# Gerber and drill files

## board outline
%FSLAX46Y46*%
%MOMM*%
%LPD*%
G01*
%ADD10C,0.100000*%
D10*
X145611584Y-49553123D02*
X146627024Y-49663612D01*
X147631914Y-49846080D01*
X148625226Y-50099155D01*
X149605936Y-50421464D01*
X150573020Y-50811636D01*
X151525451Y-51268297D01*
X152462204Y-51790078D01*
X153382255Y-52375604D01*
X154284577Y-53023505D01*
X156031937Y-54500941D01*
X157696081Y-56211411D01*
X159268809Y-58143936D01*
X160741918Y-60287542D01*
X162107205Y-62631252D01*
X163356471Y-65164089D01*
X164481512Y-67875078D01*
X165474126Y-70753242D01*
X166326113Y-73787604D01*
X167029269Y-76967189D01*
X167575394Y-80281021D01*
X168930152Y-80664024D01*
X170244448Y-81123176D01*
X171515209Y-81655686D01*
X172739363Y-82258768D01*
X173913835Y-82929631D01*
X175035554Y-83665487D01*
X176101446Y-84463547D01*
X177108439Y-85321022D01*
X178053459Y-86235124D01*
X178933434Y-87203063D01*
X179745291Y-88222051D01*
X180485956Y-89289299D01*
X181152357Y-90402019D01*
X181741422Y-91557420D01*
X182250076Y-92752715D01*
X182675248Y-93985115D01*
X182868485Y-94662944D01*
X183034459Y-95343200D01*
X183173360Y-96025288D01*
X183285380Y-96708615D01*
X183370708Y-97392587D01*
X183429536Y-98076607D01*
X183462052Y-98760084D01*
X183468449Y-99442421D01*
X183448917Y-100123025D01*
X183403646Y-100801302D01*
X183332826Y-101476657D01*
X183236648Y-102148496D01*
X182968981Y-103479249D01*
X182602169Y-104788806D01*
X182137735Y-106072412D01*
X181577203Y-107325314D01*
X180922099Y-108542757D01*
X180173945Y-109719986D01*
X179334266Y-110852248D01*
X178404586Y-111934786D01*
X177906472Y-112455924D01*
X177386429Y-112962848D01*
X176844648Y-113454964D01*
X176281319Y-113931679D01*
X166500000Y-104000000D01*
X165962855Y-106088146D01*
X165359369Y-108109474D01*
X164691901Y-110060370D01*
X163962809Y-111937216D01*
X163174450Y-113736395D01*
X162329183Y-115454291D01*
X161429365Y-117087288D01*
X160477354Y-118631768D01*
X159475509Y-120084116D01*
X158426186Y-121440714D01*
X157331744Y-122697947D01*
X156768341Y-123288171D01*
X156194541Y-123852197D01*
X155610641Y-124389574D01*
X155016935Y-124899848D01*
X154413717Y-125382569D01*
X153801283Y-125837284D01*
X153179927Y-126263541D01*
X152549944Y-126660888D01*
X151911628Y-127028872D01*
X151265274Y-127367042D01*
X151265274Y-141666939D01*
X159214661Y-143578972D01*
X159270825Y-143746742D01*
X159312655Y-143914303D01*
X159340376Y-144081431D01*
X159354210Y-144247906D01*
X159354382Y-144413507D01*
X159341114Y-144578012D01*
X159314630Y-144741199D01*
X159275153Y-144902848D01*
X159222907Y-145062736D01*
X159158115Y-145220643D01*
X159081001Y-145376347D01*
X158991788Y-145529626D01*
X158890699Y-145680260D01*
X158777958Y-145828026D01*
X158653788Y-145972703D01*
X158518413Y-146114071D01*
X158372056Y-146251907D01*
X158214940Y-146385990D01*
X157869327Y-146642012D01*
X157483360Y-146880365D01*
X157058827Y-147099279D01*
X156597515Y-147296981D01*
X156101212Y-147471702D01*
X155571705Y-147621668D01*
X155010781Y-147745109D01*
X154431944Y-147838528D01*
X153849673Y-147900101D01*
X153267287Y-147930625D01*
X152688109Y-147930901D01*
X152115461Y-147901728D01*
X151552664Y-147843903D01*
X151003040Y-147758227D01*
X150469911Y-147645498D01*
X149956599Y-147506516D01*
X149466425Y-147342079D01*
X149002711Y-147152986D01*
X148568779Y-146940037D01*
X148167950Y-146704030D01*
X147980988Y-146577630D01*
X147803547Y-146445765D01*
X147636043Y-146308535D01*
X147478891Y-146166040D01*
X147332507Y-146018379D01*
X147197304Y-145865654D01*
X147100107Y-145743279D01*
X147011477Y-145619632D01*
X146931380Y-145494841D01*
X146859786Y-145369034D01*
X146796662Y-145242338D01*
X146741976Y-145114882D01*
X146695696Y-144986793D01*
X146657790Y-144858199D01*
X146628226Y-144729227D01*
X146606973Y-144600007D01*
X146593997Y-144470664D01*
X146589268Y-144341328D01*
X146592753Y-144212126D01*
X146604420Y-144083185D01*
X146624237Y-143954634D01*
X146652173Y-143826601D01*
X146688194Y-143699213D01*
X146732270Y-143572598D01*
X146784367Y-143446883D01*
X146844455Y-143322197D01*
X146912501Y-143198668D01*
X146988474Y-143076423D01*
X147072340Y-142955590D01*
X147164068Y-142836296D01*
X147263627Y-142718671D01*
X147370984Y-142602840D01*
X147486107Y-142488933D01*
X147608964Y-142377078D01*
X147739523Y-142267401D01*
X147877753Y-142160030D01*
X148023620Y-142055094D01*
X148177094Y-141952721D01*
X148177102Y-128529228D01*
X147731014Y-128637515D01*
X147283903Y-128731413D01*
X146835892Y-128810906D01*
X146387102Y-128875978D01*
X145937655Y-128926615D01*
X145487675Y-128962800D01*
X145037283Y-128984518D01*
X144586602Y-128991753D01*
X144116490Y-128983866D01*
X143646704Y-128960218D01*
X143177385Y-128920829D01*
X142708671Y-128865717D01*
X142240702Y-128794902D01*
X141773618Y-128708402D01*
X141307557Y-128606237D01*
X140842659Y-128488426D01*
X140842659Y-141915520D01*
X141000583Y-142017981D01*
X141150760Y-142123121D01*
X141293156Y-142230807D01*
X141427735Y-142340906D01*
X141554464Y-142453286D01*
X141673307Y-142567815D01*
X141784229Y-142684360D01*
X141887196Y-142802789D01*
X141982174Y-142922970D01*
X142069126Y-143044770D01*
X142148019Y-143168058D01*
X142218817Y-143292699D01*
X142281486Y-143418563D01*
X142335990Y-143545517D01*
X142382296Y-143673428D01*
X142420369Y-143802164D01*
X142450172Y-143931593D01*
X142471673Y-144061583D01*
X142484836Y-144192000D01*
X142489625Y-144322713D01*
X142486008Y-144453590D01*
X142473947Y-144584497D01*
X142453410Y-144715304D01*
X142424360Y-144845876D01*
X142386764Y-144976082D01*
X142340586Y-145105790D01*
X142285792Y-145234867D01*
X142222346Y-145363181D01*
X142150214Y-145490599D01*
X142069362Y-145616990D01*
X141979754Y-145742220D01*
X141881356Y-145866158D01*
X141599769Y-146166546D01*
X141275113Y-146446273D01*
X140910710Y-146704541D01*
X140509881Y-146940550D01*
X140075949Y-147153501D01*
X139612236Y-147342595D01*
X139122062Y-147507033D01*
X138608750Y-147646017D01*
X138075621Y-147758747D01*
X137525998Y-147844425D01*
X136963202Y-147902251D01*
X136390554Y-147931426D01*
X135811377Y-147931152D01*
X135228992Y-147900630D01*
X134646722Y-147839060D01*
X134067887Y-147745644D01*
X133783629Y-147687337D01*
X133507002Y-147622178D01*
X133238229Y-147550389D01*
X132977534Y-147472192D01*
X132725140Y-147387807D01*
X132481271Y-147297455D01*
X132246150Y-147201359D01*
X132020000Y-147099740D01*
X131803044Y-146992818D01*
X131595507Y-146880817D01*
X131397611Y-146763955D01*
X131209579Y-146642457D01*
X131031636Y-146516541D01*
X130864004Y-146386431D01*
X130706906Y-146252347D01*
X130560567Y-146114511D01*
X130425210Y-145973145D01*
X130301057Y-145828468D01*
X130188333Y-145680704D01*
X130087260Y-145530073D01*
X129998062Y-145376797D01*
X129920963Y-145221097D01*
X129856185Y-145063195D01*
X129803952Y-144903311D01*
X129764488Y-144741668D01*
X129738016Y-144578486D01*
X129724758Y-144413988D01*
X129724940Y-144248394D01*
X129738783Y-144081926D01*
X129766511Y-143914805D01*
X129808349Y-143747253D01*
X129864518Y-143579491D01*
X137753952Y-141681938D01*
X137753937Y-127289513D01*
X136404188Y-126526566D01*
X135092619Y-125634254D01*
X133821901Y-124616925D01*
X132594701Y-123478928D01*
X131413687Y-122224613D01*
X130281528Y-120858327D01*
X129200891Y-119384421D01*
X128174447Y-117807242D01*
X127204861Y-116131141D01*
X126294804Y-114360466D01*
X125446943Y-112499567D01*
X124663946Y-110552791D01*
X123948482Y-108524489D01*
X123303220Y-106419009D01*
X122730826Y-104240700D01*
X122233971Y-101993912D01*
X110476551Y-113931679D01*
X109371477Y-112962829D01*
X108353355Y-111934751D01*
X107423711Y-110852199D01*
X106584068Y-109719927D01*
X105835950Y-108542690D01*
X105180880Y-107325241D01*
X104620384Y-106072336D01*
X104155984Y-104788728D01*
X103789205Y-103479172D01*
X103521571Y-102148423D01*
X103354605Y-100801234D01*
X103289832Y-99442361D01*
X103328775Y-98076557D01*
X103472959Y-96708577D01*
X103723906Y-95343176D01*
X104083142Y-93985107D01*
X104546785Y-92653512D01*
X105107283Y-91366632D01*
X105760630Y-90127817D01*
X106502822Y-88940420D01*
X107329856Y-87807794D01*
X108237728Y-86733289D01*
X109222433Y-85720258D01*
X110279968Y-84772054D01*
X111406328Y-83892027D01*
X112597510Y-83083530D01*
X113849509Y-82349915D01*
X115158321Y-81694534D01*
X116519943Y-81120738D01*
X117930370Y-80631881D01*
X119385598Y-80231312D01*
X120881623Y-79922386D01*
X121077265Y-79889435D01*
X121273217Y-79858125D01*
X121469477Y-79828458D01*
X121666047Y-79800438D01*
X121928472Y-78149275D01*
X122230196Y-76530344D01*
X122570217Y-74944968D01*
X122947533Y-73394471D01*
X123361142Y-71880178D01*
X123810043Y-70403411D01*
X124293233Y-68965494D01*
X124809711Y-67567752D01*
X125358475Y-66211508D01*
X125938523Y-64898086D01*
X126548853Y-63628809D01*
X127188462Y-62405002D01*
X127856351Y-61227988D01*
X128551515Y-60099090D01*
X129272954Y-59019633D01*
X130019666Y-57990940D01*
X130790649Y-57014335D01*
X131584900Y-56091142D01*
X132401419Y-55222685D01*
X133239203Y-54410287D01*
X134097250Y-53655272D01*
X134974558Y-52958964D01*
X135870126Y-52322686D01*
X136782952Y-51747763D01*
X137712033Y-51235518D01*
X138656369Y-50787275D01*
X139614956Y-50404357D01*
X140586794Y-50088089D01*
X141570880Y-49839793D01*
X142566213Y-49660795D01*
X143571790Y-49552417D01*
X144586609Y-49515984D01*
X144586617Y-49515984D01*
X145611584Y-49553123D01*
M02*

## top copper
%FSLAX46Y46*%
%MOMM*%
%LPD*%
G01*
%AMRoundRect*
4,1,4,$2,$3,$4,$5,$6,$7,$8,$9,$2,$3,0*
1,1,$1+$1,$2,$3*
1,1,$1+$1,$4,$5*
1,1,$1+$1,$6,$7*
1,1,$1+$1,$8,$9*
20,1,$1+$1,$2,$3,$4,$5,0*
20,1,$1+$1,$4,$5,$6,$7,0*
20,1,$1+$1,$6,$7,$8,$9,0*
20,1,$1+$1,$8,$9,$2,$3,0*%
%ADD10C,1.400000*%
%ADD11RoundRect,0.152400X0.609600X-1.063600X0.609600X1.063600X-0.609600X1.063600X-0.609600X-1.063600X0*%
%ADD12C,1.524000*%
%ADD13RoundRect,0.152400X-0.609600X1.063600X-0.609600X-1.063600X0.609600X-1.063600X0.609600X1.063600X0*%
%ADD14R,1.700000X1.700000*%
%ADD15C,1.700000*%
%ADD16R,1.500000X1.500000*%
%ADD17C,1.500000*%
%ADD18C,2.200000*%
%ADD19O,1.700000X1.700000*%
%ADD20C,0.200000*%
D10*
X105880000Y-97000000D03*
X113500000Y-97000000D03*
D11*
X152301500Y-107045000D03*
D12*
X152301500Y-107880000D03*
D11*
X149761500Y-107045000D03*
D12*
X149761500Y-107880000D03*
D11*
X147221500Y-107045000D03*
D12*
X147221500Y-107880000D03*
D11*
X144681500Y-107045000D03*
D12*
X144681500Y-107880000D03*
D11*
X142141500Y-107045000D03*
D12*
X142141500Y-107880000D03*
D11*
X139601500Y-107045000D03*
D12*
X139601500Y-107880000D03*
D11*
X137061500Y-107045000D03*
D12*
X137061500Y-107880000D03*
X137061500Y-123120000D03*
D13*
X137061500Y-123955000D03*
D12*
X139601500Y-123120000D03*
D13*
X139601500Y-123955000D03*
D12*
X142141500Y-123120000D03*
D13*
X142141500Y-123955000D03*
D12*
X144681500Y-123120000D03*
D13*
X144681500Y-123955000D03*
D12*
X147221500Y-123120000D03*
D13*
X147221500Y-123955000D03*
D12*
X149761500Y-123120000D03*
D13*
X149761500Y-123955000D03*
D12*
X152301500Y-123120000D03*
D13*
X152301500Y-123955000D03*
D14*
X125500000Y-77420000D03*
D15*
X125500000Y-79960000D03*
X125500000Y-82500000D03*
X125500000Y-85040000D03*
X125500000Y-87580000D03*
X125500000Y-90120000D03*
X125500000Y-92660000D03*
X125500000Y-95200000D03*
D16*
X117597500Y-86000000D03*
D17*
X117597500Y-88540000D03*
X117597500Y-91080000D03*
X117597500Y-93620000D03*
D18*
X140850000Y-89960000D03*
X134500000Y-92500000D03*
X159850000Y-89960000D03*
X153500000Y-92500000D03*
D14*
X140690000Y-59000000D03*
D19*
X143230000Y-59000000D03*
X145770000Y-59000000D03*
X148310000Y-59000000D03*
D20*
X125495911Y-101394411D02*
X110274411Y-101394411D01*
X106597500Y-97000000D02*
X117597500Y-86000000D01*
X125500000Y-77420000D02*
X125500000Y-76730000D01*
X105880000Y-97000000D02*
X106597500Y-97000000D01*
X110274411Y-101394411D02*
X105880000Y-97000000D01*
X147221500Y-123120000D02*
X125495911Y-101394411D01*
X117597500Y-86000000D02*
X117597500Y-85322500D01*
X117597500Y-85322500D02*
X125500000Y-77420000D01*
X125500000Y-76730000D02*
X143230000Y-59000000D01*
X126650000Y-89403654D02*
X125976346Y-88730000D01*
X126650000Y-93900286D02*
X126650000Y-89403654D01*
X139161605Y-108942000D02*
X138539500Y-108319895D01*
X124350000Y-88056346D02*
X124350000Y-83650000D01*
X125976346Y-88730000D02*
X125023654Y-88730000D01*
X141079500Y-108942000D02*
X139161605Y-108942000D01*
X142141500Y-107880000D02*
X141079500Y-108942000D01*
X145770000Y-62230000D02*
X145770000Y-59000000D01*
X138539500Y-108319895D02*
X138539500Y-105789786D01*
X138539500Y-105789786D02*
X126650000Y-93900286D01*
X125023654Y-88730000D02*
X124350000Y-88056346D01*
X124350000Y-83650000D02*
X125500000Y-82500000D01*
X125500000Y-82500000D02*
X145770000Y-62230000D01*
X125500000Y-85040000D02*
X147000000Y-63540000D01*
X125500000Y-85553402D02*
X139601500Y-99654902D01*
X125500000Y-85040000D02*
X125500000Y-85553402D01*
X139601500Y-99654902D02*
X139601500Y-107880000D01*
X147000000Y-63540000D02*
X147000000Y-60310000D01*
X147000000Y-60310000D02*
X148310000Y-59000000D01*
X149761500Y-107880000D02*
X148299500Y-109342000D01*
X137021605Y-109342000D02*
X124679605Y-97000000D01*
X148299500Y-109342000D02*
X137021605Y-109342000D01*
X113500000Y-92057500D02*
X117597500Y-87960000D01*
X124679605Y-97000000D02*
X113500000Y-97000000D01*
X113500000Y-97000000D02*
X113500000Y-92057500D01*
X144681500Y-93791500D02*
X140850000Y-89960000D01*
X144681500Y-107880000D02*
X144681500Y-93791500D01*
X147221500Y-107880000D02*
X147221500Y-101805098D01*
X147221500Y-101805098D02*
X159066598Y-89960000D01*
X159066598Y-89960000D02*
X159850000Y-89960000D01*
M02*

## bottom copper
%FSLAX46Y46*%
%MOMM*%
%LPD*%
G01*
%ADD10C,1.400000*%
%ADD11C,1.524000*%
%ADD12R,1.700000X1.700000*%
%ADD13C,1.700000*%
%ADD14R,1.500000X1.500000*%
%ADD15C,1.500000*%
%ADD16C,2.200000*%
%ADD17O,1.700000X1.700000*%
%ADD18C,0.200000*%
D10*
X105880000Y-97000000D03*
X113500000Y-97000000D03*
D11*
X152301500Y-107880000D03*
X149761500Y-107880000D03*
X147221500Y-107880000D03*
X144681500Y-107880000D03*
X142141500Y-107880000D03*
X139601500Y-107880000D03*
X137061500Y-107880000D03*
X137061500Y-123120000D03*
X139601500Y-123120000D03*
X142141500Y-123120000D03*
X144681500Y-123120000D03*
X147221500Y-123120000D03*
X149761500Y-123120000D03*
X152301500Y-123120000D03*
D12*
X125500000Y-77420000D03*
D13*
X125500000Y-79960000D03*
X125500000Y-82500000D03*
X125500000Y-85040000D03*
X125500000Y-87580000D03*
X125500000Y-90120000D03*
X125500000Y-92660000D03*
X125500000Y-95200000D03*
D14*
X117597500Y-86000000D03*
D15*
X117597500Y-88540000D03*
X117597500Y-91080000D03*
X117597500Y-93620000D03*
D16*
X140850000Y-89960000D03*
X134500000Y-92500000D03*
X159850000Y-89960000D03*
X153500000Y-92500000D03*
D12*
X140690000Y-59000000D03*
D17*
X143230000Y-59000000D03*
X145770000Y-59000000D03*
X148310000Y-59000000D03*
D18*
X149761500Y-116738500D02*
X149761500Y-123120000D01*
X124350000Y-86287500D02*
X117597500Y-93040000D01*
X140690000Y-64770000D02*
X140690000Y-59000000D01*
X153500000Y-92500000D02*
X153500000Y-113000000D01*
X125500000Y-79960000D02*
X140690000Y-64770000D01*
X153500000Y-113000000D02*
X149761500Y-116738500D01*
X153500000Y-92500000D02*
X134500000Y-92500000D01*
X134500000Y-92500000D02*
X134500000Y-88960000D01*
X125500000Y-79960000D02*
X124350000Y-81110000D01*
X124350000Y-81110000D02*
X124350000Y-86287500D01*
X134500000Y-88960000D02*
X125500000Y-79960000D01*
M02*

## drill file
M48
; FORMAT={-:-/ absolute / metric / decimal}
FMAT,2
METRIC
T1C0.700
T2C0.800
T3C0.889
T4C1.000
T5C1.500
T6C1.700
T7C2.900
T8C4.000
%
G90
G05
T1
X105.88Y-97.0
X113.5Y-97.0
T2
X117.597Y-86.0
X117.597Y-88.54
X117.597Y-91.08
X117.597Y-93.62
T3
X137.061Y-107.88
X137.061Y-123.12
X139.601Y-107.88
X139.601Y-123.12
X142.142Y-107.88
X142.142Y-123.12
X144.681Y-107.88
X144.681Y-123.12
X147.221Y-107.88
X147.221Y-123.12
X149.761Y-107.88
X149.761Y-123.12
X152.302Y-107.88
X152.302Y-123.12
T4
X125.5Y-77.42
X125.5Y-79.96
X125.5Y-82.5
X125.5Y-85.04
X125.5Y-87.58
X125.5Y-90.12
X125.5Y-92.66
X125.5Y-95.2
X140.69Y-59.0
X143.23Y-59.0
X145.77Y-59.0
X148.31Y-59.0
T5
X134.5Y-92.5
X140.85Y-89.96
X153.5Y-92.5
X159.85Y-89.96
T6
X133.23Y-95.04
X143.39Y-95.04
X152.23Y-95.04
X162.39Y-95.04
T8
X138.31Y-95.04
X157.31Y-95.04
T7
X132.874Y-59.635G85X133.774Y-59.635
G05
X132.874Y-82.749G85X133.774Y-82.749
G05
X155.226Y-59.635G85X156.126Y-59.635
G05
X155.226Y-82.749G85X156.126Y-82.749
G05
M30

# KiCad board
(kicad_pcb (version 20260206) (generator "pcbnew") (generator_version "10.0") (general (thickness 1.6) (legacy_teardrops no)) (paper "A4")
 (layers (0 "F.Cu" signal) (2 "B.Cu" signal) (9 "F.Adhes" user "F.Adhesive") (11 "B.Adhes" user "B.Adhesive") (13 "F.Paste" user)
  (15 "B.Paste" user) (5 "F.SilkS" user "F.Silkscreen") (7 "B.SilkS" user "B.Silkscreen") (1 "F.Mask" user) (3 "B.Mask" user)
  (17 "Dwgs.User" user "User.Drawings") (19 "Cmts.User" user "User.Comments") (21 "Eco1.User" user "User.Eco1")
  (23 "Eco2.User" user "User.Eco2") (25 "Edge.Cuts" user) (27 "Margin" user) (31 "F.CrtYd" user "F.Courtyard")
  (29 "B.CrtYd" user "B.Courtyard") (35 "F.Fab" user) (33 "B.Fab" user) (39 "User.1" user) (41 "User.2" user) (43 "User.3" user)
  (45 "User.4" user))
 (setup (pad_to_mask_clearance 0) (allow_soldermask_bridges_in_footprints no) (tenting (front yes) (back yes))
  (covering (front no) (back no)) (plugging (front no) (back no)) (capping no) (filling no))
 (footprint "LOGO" (layer "F.Cu") (at 143 97)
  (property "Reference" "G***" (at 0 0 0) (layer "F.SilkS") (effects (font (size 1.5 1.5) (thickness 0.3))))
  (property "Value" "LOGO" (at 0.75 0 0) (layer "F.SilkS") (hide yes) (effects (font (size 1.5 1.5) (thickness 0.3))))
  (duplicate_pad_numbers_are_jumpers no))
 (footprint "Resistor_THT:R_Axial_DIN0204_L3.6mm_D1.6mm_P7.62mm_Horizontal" (layer "F.Cu") (at 105.88 97)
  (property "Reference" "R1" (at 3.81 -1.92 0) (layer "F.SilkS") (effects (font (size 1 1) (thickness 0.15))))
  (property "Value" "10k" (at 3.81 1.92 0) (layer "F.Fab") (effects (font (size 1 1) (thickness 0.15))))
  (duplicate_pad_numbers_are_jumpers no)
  (pad "1" thru_hole circle (at 0 0) (size 1.4 1.4) (drill 0.7) (layers "*.Cu" "*.Mask") (remove_unused_layers no) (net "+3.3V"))
  (pad "2" thru_hole circle (at 7.62 0) (size 1.4 1.4) (drill 0.7) (layers "*.Cu" "*.Mask") (remove_unused_layers no) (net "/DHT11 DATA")))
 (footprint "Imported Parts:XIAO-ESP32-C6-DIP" (layer "F.Cu") (at 144.6815 115.5)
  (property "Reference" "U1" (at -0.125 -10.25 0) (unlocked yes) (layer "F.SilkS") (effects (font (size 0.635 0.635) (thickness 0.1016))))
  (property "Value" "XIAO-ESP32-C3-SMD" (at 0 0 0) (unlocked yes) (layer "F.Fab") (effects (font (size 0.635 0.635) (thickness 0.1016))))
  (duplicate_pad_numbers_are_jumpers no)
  (pad "1" smd roundrect (at 7.62 -8.455 90) (size 2.432 1.524) (layers "F.Cu" "F.Mask") (roundrect_rratio 0.1)
   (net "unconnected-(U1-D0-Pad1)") (thermal_bridge_angle 45))
  (pad "1" thru_hole circle (at 7.62 -7.62 90) (size 1.524 1.524) (drill 0.889) (layers "*.Cu" "*.Mask") (remove_unused_layers no)
   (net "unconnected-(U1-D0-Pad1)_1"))
  (pad "2" smd roundrect (at 5.08 -8.455 90) (size 2.432 1.524) (layers "F.Cu" "F.Mask") (roundrect_rratio 0.1) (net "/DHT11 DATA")
   (thermal_bridge_angle 45))
  (pad "2" thru_hole circle (at 5.08 -7.62 90) (size 1.524 1.524) (drill 0.889) (layers "*.Cu" "*.Mask") (remove_unused_layers no)
   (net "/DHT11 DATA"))
  (pad "3" smd roundrect (at 2.54 -8.455 90) (size 2.432 1.524) (layers "F.Cu" "F.Mask") (roundrect_rratio 0.1) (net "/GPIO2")
   (thermal_bridge_angle 45))
  (pad "3" thru_hole circle (at 2.54 -7.62 90) (size 1.524 1.524) (drill 0.889) (layers "*.Cu" "*.Mask") (remove_unused_layers no)
   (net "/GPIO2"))
  (pad "4" smd roundrect (at 0 -8.455 90) (size 2.432 1.524) (layers "F.Cu" "F.Mask") (roundrect_rratio 0.1) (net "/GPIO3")
   (thermal_bridge_angle 45))
  (pad "4" thru_hole circle (at 0 -7.62 90) (size 1.524 1.524) (drill 0.889) (layers "*.Cu" "*.Mask") (remove_unused_layers no)
   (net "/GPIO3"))
  (pad "5" smd roundrect (at -2.54 -8.455 90) (size 2.432 1.524) (layers "F.Cu" "F.Mask") (roundrect_rratio 0.1) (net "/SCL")
   (thermal_bridge_angle 45))
  (pad "5" thru_hole circle (at -2.54 -7.62 90) (size 1.524 1.524) (drill 0.889) (layers "*.Cu" "*.Mask") (remove_unused_layers no)
   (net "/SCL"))
  (pad "6" smd roundrect (at -5.08 -8.455 90) (size 2.432 1.524) (layers "F.Cu" "F.Mask") (roundrect_rratio 0.1) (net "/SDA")
   (thermal_bridge_angle 45))
  (pad "6" thru_hole circle (at -5.08 -7.62 90) (size 1.524 1.524) (drill 0.889) (layers "*.Cu" "*.Mask") (remove_unused_layers no)
   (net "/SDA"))
  (pad "7" smd roundrect (at -7.62 -8.455 90) (size 2.432 1.524) (layers "F.Cu" "F.Mask") (roundrect_rratio 0.1)
   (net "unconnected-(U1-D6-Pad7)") (thermal_bridge_angle 45))
  (pad "7" thru_hole circle (at -7.62 -7.62 90) (size 1.524 1.524) (drill 0.889) (layers "*.Cu" "*.Mask") (remove_unused_layers no)
   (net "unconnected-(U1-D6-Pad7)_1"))
  (pad "8" thru_hole circle (at -7.62 7.62 270) (size 1.524 1.524) (drill 0.889) (layers "*.Cu" "*.Mask") (remove_unused_layers no)
   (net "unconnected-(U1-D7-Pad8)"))
  (pad "8" smd roundrect (at -7.62 8.455 270) (size 2.432 1.524) (layers "F.Cu" "F.Mask") (roundrect_rratio 0.1)
   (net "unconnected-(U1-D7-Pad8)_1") (thermal_bridge_angle 45))
  (pad "9" thru_hole circle (at -5.08 7.62 270) (size 1.524 1.524) (drill 0.889) (layers "*.Cu" "*.Mask") (remove_unused_layers no)
   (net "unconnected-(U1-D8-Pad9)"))
  (pad "9" smd roundrect (at -5.08 8.455 270) (size 2.432 1.524) (layers "F.Cu" "F.Mask") (roundrect_rratio 0.1)
   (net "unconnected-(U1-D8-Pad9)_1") (thermal_bridge_angle 45))
  (pad "10" thru_hole circle (at -2.54 7.62 270) (size 1.524 1.524) (drill 0.889) (layers "*.Cu" "*.Mask") (remove_unused_layers no)
   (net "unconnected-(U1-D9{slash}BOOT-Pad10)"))
  (pad "10" smd roundrect (at -2.54 8.455 270) (size 2.432 1.524) (layers "F.Cu" "F.Mask") (roundrect_rratio 0.1)
   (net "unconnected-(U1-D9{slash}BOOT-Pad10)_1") (thermal_bridge_angle 45))
  (pad "11" thru_hole circle (at 0 7.62 270) (size 1.524 1.524) (drill 0.889) (layers "*.Cu" "*.Mask") (remove_unused_layers no)
   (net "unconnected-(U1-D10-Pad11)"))
  (pad "11" smd roundrect (at 0 8.455 270) (size 2.432 1.524) (layers "F.Cu" "F.Mask") (roundrect_rratio 0.1)
   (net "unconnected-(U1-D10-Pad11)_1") (thermal_bridge_angle 45))
  (pad "12" thru_hole circle (at 2.54 7.62 270) (size 1.524 1.524) (drill 0.889) (layers "*.Cu" "*.Mask") (remove_unused_layers no)
   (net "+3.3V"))
  (pad "12" smd roundrect (at 2.54 8.455 270) (size 2.432 1.524) (layers "F.Cu" "F.Mask") (roundrect_rratio 0.1) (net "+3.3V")
   (thermal_bridge_angle 45))
  (pad "13" thru_hole circle (at 5.08 7.62 270) (size 1.524 1.524) (drill 0.889) (layers "*.Cu" "*.Mask") (remove_unused_layers no)
   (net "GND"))
  (pad "13" smd roundrect (at 5.08 8.455 270) (size 2.432 1.524) (layers "F.Cu" "F.Mask") (roundrect_rratio 0.1) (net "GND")
   (thermal_bridge_angle 45))
  (pad "14" thru_hole circle (at 7.62 7.62 270) (size 1.524 1.524) (drill 0.889) (layers "*.Cu" "*.Mask") (remove_unused_layers no)
   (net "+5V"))
  (pad "14" smd roundrect (at 7.62 8.455 270) (size 2.432 1.524) (layers "F.Cu" "F.Mask") (roundrect_rratio 0.1) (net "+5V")
   (thermal_bridge_angle 45)))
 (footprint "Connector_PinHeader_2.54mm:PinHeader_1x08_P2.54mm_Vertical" (layer "F.Cu") (at 125.5 77.42)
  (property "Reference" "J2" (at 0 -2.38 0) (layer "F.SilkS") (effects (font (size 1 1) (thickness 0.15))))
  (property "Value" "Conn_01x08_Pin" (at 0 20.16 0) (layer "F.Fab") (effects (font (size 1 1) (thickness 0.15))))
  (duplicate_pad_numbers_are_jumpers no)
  (pad "1" thru_hole rect (at 0 0) (size 1.7 1.7) (drill 1) (layers "*.Cu" "*.Mask") (remove_unused_layers no) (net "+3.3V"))
  (pad "2" thru_hole circle (at 0 2.54) (size 1.7 1.7) (drill 1) (layers "*.Cu" "*.Mask") (remove_unused_layers no) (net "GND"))
  (pad "3" thru_hole circle (at 0 5.08) (size 1.7 1.7) (drill 1) (layers "*.Cu" "*.Mask") (remove_unused_layers no) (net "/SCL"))
  (pad "4" thru_hole circle (at 0 7.62) (size 1.7 1.7) (drill 1) (layers "*.Cu" "*.Mask") (remove_unused_layers no) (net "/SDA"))
  (pad "5" thru_hole circle (at 0 10.16) (size 1.7 1.7) (drill 1) (layers "*.Cu" "*.Mask") (remove_unused_layers no)
   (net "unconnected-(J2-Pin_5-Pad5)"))
  (pad "6" thru_hole circle (at 0 12.7) (size 1.7 1.7) (drill 1) (layers "*.Cu" "*.Mask") (remove_unused_layers no)
   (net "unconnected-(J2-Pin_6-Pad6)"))
  (pad "7" thru_hole circle (at 0 15.24) (size 1.7 1.7) (drill 1) (layers "*.Cu" "*.Mask") (remove_unused_layers no)
   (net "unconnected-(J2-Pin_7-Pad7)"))
  (pad "8" thru_hole circle (at 0 17.78) (size 1.7 1.7) (drill 1) (layers "*.Cu" "*.Mask") (remove_unused_layers no)
   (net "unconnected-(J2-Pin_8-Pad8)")))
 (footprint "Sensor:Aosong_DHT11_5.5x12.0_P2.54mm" (layer "F.Cu") (at 117.5975 86)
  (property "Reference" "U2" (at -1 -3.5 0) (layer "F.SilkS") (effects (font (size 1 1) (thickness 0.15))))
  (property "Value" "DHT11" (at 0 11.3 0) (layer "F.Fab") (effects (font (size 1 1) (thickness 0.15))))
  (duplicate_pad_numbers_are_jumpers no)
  (pad "1" thru_hole rect (at 0 0) (size 1.5 1.5) (drill 0.8) (layers "*.Cu" "*.Mask") (remove_unused_layers no) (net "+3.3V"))
  (pad "2" thru_hole circle (at 0 2.54) (size 1.5 1.5) (drill 0.8) (layers "*.Cu" "*.Mask") (remove_unused_layers no) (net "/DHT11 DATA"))
  (pad "3" thru_hole circle (at 0 5.08) (size 1.5 1.5) (drill 0.8) (layers "*.Cu" "*.Mask") (remove_unused_layers no)
   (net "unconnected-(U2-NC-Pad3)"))
  (pad "4" thru_hole circle (at 0 7.62) (size 1.5 1.5) (drill 0.8) (layers "*.Cu" "*.Mask") (remove_unused_layers no) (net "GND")))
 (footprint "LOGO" (layer "F.Cu") (at 142.5 98.5)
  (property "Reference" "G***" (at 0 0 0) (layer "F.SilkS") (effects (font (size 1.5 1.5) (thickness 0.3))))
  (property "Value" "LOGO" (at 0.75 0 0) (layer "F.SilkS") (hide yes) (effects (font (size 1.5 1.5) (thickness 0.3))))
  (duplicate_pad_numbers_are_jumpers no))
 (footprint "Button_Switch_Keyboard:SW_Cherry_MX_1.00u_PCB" (layer "F.Cu") (at 140.85 89.96)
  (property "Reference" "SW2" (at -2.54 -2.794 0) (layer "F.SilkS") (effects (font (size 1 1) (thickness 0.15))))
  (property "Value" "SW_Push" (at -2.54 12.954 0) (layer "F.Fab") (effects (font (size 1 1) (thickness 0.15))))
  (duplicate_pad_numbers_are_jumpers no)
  (pad "" np_thru_hole circle (at -7.62 5.08) (size 1.7 1.7) (drill 1.7) (layers "*.Cu" "*.Mask"))
  (pad "" np_thru_hole circle (at -2.54 5.08) (size 4 4) (drill 4) (layers "*.Cu" "*.Mask"))
  (pad "" np_thru_hole circle (at 2.54 5.08) (size 1.7 1.7) (drill 1.7) (layers "*.Cu" "*.Mask"))
  (pad "1" thru_hole circle (at 0 0) (size 2.2 2.2) (drill 1.5) (layers "*.Cu" "*.Mask") (remove_unused_layers no) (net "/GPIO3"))
  (pad "2" thru_hole circle (at -6.35 2.54) (size 2.2 2.2) (drill 1.5) (layers "*.Cu" "*.Mask") (remove_unused_layers no) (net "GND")))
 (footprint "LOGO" (layer "F.Cu") (at 143 98.5)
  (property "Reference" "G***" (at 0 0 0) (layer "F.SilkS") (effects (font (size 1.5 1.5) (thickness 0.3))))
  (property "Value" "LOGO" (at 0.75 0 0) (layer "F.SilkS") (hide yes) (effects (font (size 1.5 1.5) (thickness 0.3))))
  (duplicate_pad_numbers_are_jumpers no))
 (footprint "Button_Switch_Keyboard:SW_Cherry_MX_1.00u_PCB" (layer "F.Cu") (at 159.85 89.96)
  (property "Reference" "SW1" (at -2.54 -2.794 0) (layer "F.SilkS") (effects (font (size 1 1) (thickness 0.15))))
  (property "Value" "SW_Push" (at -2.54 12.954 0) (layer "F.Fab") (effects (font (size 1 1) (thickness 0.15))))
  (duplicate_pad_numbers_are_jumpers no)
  (pad "" np_thru_hole circle (at -7.62 5.08) (size 1.7 1.7) (drill 1.7) (layers "*.Cu" "*.Mask"))
  (pad "" np_thru_hole circle (at -2.54 5.08) (size 4 4) (drill 4) (layers "*.Cu" "*.Mask"))
  (pad "" np_thru_hole circle (at 2.54 5.08) (size 1.7 1.7) (drill 1.7) (layers "*.Cu" "*.Mask"))
  (pad "1" thru_hole circle (at 0 0) (size 2.2 2.2) (drill 1.5) (layers "*.Cu" "*.Mask") (remove_unused_layers no) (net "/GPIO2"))
  (pad "2" thru_hole circle (at -6.35 2.54) (size 2.2 2.2) (drill 1.5) (layers "*.Cu" "*.Mask") (remove_unused_layers no) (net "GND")))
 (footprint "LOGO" (layer "F.Cu") (at 142.5 97.5)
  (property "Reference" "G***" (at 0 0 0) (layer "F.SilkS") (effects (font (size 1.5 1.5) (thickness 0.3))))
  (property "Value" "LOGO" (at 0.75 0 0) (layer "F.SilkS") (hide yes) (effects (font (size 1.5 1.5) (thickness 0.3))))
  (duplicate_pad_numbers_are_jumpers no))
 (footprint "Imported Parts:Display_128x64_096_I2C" (layer "F.Cu") (at 144.5 59)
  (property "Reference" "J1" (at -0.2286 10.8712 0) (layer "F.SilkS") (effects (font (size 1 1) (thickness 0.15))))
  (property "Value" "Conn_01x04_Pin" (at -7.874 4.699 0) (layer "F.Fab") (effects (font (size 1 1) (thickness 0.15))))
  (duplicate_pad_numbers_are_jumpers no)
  (pad "" np_thru_hole oval (at -11.176 0.635) (size 3.8 2.9) (drill oval 3.8 2.9) (layers "*.Cu" "*.Mask"))
  (pad "" np_thru_hole oval (at -11.176 23.749) (size 3.8 2.9) (drill oval 3.8 2.9) (layers "*.Cu" "*.Mask"))
  (pad "" np_thru_hole oval (at 11.176 0.635) (size 3.8 2.9) (drill oval 3.8 2.9) (layers "*.Cu" "*.Mask"))
  (pad "" np_thru_hole oval (at 11.176 23.749) (size 3.8 2.9) (drill oval 3.8 2.9) (layers "*.Cu" "*.Mask"))
  (pad "1" thru_hole rect (at -3.81 0 90) (size 1.7 1.7) (drill 1) (layers "*.Cu" "*.Mask") (remove_unused_layers no) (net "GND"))
  (pad "2" thru_hole oval (at -1.27 0 90) (size 1.7 1.7) (drill 1) (layers "*.Cu" "*.Mask") (remove_unused_layers no) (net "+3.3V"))
  (pad "3" thru_hole oval (at 1.27 0 90) (size 1.7 1.7) (drill 1) (layers "*.Cu" "*.Mask") (remove_unused_layers no) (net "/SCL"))
  (pad "4" thru_hole oval (at 3.81 0 90) (size 1.7 1.7) (drill 1) (layers "*.Cu" "*.Mask") (remove_unused_layers no) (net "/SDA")))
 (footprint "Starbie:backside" (layer "B.Cu") (at 145 96.5 180)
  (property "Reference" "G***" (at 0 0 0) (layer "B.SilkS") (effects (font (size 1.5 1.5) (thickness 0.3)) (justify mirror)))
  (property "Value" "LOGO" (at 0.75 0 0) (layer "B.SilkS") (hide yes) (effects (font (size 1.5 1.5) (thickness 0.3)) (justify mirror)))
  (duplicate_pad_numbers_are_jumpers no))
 (gr_poly
  (pts (xy 145.611584 49.553123) (xy 146.627024 49.663612) (xy 147.631914 49.84608) (xy 148.625226 50.099155) (xy 149.605936 50.421464)
   (xy 150.57302 50.811636) (xy 151.525451 51.268297) (xy 152.462204 51.790078) (xy 153.382255 52.375604) (xy 154.284577 53.023505)
   (xy 156.031937 54.500941) (xy 157.696081 56.211411) (xy 159.268809 58.143936) (xy 160.741918 60.287542) (xy 162.107205 62.631252)
   (xy 163.356471 65.164089) (xy 164.481512 67.875078) (xy 165.474126 70.753242) (xy 166.326113 73.787604) (xy 167.029269 76.967189)
   (xy 167.575394 80.281021) (xy 168.930152 80.664024) (xy 170.244448 81.123176) (xy 171.515209 81.655686) (xy 172.739363 82.258768)
   (xy 173.913835 82.929631) (xy 175.035554 83.665487) (xy 176.101446 84.463547) (xy 177.108439 85.321022) (xy 178.053459 86.235124)
   (xy 178.933434 87.203063) (xy 179.745291 88.222051) (xy 180.485956 89.289299) (xy 181.152357 90.402019) (xy 181.741422 91.55742)
   (xy 182.250076 92.752715) (xy 182.675248 93.985115) (xy 182.868485 94.662944) (xy 183.034459 95.3432) (xy 183.17336 96.025288)
   (xy 183.28538 96.708615) (xy 183.370708 97.392587) (xy 183.429536 98.076607) (xy 183.462052 98.760084) (xy 183.468449 99.442421)
   (xy 183.448917 100.123025) (xy 183.403646 100.801302) (xy 183.332826 101.476657) (xy 183.236648 102.148496) (xy 182.968981 103.479249)
   (xy 182.602169 104.788806) (xy 182.137735 106.072412) (xy 181.577203 107.325314) (xy 180.922099 108.542757) (xy 180.173945 109.719986)
   (xy 179.334266 110.852248) (xy 178.404586 111.934786) (xy 177.906472 112.455924) (xy 177.386429 112.962848) (xy 176.844648 113.454964)
   (xy 176.281319 113.931679) (xy 166.5 104) (xy 165.962855 106.088146) (xy 165.359369 108.109474) (xy 164.691901 110.06037)
   (xy 163.962809 111.937216) (xy 163.17445 113.736395) (xy 162.329183 115.454291) (xy 161.429365 117.087288) (xy 160.477354 118.631768)
   (xy 159.475509 120.084116) (xy 158.426186 121.440714) (xy 157.331744 122.697947) (xy 156.768341 123.288171) (xy 156.194541 123.852197)
   (xy 155.610641 124.389574) (xy 155.016935 124.899848) (xy 154.413717 125.382569) (xy 153.801283 125.837284) (xy 153.179927 126.263541)
   (xy 152.549944 126.660888) (xy 151.911628 127.028872) (xy 151.265274 127.367042) (xy 151.265274 141.666939) (xy 159.214661 143.578972)
   (xy 159.270825 143.746742) (xy 159.312655 143.914303) (xy 159.340376 144.081431) (xy 159.35421 144.247906) (xy 159.354382 144.413507)
   (xy 159.341114 144.578012) (xy 159.31463 144.741199) (xy 159.275153 144.902848) (xy 159.222907 145.062736) (xy 159.158115 145.220643)
   (xy 159.081001 145.376347) (xy 158.991788 145.529626) (xy 158.890699 145.68026) (xy 158.777958 145.828026) (xy 158.653788 145.972703)
   (xy 158.518413 146.114071) (xy 158.372056 146.251907) (xy 158.21494 146.38599) (xy 157.869327 146.642012) (xy 157.48336 146.880365)
   (xy 157.058827 147.099279) (xy 156.597515 147.296981) (xy 156.101212 147.471702) (xy 155.571705 147.621668) (xy 155.010781 147.745109)
   (xy 154.431944 147.838528) (xy 153.849673 147.900101) (xy 153.267287 147.930625) (xy 152.688109 147.930901) (xy 152.115461 147.901728)
   (xy 151.552664 147.843903) (xy 151.00304 147.758227) (xy 150.469911 147.645498) (xy 149.956599 147.506516) (xy 149.466425 147.342079)
   (xy 149.002711 147.152986) (xy 148.568779 146.940037) (xy 148.16795 146.70403) (xy 147.980988 146.57763) (xy 147.803547 146.445765)
   (xy 147.636043 146.308535) (xy 147.478891 146.16604) (xy 147.332507 146.018379) (xy 147.197304 145.865654) (xy 147.100107 145.743279)
   (xy 147.011477 145.619632) (xy 146.93138 145.494841) (xy 146.859786 145.369034) (xy 146.796662 145.242338) (xy 146.741976 145.114882)
   (xy 146.695696 144.986793) (xy 146.65779 144.858199) (xy 146.628226 144.729227) (xy 146.606973 144.600007) (xy 146.593997 144.470664)
   (xy 146.589268 144.341328) (xy 146.592753 144.212126) (xy 146.60442 144.083185) (xy 146.624237 143.954634) (xy 146.652173 143.826601)
   (xy 146.688194 143.699213) (xy 146.73227 143.572598) (xy 146.784367 143.446883) (xy 146.844455 143.322197) (xy 146.912501 143.198668)
   (xy 146.988474 143.076423) (xy 147.07234 142.95559) (xy 147.164068 142.836296) (xy 147.263627 142.718671) (xy 147.370984 142.60284)
   (xy 147.486107 142.488933) (xy 147.608964 142.377078) (xy 147.739523 142.267401) (xy 147.877753 142.16003) (xy 148.02362 142.055094)
   (xy 148.177094 141.952721) (xy 148.177102 128.529228) (xy 147.731014 128.637515) (xy 147.283903 128.731413) (xy 146.835892 128.810906)
   (xy 146.387102 128.875978) (xy 145.937655 128.926615) (xy 145.487675 128.9628) (xy 145.037283 128.984518) (xy 144.586602 128.991753)
   (xy 144.11649 128.983866) (xy 143.646704 128.960218) (xy 143.177385 128.920829) (xy 142.708671 128.865717) (xy 142.240702 128.794902)
   (xy 141.773618 128.708402) (xy 141.307557 128.606237) (xy 140.842659 128.488426) (xy 140.842659 141.91552) (xy 141.000583 142.017981)
   (xy 141.15076 142.123121) (xy 141.293156 142.230807) (xy 141.427735 142.340906) (xy 141.554464 142.453286) (xy 141.673307 142.567815)
   (xy 141.784229 142.68436) (xy 141.887196 142.802789) (xy 141.982174 142.92297) (xy 142.069126 143.04477) (xy 142.148019 143.168058)
   (xy 142.218817 143.292699) (xy 142.281486 143.418563) (xy 142.33599 143.545517) (xy 142.382296 143.673428) (xy 142.420369 143.802164)
   (xy 142.450172 143.931593) (xy 142.471673 144.061583) (xy 142.484836 144.192) (xy 142.489625 144.322713) (xy 142.486008 144.45359)
   (xy 142.473947 144.584497) (xy 142.45341 144.715304) (xy 142.42436 144.845876) (xy 142.386764 144.976082) (xy 142.340586 145.10579)
   (xy 142.285792 145.234867) (xy 142.222346 145.363181) (xy 142.150214 145.490599) (xy 142.069362 145.61699) (xy 141.979754 145.74222)
   (xy 141.881356 145.866158) (xy 141.599769 146.166546) (xy 141.275113 146.446273) (xy 140.91071 146.704541) (xy 140.509881 146.94055)
   (xy 140.075949 147.153501) (xy 139.612236 147.342595) (xy 139.122062 147.507033) (xy 138.60875 147.646017) (xy 138.075621 147.758747)
   (xy 137.525998 147.844425) (xy 136.963202 147.902251) (xy 136.390554 147.931426) (xy 135.811377 147.931152) (xy 135.228992 147.90063)
   (xy 134.646722 147.83906) (xy 134.067887 147.745644) (xy 133.783629 147.687337) (xy 133.507002 147.622178) (xy 133.238229 147.550389)
   (xy 132.977534 147.472192) (xy 132.72514 147.387807) (xy 132.481271 147.297455) (xy 132.24615 147.201359) (xy 132.02 147.09974)
   (xy 131.803044 146.992818) (xy 131.595507 146.880817) (xy 131.397611 146.763955) (xy 131.209579 146.642457) (xy 131.031636 146.516541)
   (xy 130.864004 146.386431) (xy 130.706906 146.252347) (xy 130.560567 146.114511) (xy 130.42521 145.973145) (xy 130.301057 145.828468)
   (xy 130.188333 145.680704) (xy 130.08726 145.530073) (xy 129.998062 145.376797) (xy 129.920963 145.221097) (xy 129.856185 145.063195)
   (xy 129.803952 144.903311) (xy 129.764488 144.741668) (xy 129.738016 144.578486) (xy 129.724758 144.413988) (xy 129.72494 144.248394)
   (xy 129.738783 144.081926) (xy 129.766511 143.914805) (xy 129.808349 143.747253) (xy 129.864518 143.579491) (xy 137.753952 141.681938)
   (xy 137.753937 127.289513) (xy 136.404188 126.526566) (xy 135.092619 125.634254) (xy 133.821901 124.616925) (xy 132.594701 123.478928)
   (xy 131.413687 122.224613) (xy 130.281528 120.858327) (xy 129.200891 119.384421) (xy 128.174447 117.807242) (xy 127.204861 116.131141)
   (xy 126.294804 114.360466) (xy 125.446943 112.499567) (xy 124.663946 110.552791) (xy 123.948482 108.524489) (xy 123.30322 106.419009)
   (xy 122.730826 104.2407) (xy 122.233971 101.993912) (xy 110.476551 113.931679) (xy 109.371477 112.962829) (xy 108.353355 111.934751)
   (xy 107.423711 110.852199) (xy 106.584068 109.719927) (xy 105.83595 108.54269) (xy 105.18088 107.325241) (xy 104.620384 106.072336)
   (xy 104.155984 104.788728) (xy 103.789205 103.479172) (xy 103.521571 102.148423) (xy 103.354605 100.801234) (xy 103.289832 99.442361)
   (xy 103.328775 98.076557) (xy 103.472959 96.708577) (xy 103.723906 95.343176) (xy 104.083142 93.985107) (xy 104.546785 92.653512)
   (xy 105.107283 91.366632) (xy 105.76063 90.127817) (xy 106.502822 88.94042) (xy 107.329856 87.807794) (xy 108.237728 86.733289)
   (xy 109.222433 85.720258) (xy 110.279968 84.772054) (xy 111.406328 83.892027) (xy 112.59751 83.08353) (xy 113.849509 82.349915)
   (xy 115.158321 81.694534) (xy 116.519943 81.120738) (xy 117.93037 80.631881) (xy 119.385598 80.231312) (xy 120.881623 79.922386)
   (xy 121.077265 79.889435) (xy 121.273217 79.858125) (xy 121.469477 79.828458) (xy 121.666047 79.800438) (xy 121.928472 78.149275)
   (xy 122.230196 76.530344) (xy 122.570217 74.944968) (xy 122.947533 73.394471) (xy 123.361142 71.880178) (xy 123.810043 70.403411)
   (xy 124.293233 68.965494) (xy 124.809711 67.567752) (xy 125.358475 66.211508) (xy 125.938523 64.898086) (xy 126.548853 63.628809)
   (xy 127.188462 62.405002) (xy 127.856351 61.227988) (xy 128.551515 60.09909) (xy 129.272954 59.019633) (xy 130.019666 57.99094)
   (xy 130.790649 57.014335) (xy 131.5849 56.091142) (xy 132.401419 55.222685) (xy 133.239203 54.410287) (xy 134.09725 53.655272)
   (xy 134.974558 52.958964) (xy 135.870126 52.322686) (xy 136.782952 51.747763) (xy 137.712033 51.235518) (xy 138.656369 50.787275)
   (xy 139.614956 50.404357) (xy 140.586794 50.088089) (xy 141.57088 49.839793) (xy 142.566213 49.660795) (xy 143.57179 49.552417)
   (xy 144.586609 49.515984) (xy 144.586617 49.515984))
  (stroke (width 0.1) (type solid)) (fill no) (layer "Edge.Cuts"))
 (segment (start 149.7615 116.7385) (end 149.7615 123.12) (width 0.2) (layer "B.Cu") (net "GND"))
 (segment (start 124.35 86.2875) (end 117.5975 93.04) (width 0.2) (layer "B.Cu") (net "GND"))
 (segment (start 140.69 64.77) (end 140.69 59) (width 0.2) (layer "B.Cu") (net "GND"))
 (segment (start 153.5 92.5) (end 153.5 113) (width 0.2) (layer "B.Cu") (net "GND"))
 (segment (start 125.5 79.96) (end 140.69 64.77) (width 0.2) (layer "B.Cu") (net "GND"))
 (segment (start 153.5 113) (end 149.7615 116.7385) (width 0.2) (layer "B.Cu") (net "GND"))
 (segment (start 153.5 92.5) (end 134.5 92.5) (width 0.2) (layer "B.Cu") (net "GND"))
 (segment (start 134.5 92.5) (end 134.5 88.96) (width 0.2) (layer "B.Cu") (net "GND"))
 (segment (start 125.5 79.96) (end 124.35 81.11) (width 0.2) (layer "B.Cu") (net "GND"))
 (segment (start 124.35 81.11) (end 124.35 86.2875) (width 0.2) (layer "B.Cu") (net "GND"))
 (segment (start 134.5 88.96) (end 125.5 79.96) (width 0.2) (layer "B.Cu") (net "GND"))
 (segment (start 125.495911 101.394411) (end 110.274411 101.394411) (width 0.2) (layer "F.Cu") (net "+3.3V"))
 (segment (start 106.5975 97) (end 117.5975 86) (width 0.2) (layer "F.Cu") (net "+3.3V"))
 (segment (start 125.5 77.42) (end 125.5 76.73) (width 0.2) (layer "F.Cu") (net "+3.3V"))
 (segment (start 105.88 97) (end 106.5975 97) (width 0.2) (layer "F.Cu") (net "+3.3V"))
 (segment (start 110.274411 101.394411) (end 105.88 97) (width 0.2) (layer "F.Cu") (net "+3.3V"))
 (segment (start 147.2215 123.12) (end 125.495911 101.394411) (width 0.2) (layer "F.Cu") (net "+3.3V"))
 (segment (start 117.5975 86) (end 117.5975 85.3225) (width 0.2) (layer "F.Cu") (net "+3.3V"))
 (segment (start 117.5975 85.3225) (end 125.5 77.42) (width 0.2) (layer "F.Cu") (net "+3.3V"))
 (segment (start 125.5 76.73) (end 143.23 59) (width 0.2) (layer "F.Cu") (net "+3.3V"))
 (segment (start 126.65 89.403654) (end 125.976346 88.73) (width 0.2) (layer "F.Cu") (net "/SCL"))
 (segment (start 126.65 93.900286) (end 126.65 89.403654) (width 0.2) (layer "F.Cu") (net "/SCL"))
 (segment (start 139.161605 108.942) (end 138.5395 108.319895) (width 0.2) (layer "F.Cu") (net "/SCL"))
 (segment (start 124.35 88.056346) (end 124.35 83.65) (width 0.2) (layer "F.Cu") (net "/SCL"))
 (segment (start 125.976346 88.73) (end 125.023654 88.73) (width 0.2) (layer "F.Cu") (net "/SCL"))
 (segment (start 141.0795 108.942) (end 139.161605 108.942) (width 0.2) (layer "F.Cu") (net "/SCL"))
 (segment (start 142.1415 107.88) (end 141.0795 108.942) (width 0.2) (layer "F.Cu") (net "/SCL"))
 (segment (start 145.77 62.23) (end 145.77 59) (width 0.2) (layer "F.Cu") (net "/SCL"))
 (segment (start 138.5395 108.319895) (end 138.5395 105.789786) (width 0.2) (layer "F.Cu") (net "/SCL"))
 (segment (start 138.5395 105.789786) (end 126.65 93.900286) (width 0.2) (layer "F.Cu") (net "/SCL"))
 (segment (start 125.023654 88.73) (end 124.35 88.056346) (width 0.2) (layer "F.Cu") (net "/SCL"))
 (segment (start 124.35 83.65) (end 125.5 82.5) (width 0.2) (layer "F.Cu") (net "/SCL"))
 (segment (start 125.5 82.5) (end 145.77 62.23) (width 0.2) (layer "F.Cu") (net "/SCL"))
 (segment (start 125.5 85.04) (end 147 63.54) (width 0.2) (layer "F.Cu") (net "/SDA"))
 (segment (start 125.5 85.553402) (end 139.6015 99.654902) (width 0.2) (layer "F.Cu") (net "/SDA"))
 (segment (start 125.5 85.04) (end 125.5 85.553402) (width 0.2) (layer "F.Cu") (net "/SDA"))
 (segment (start 139.6015 99.654902) (end 139.6015 107.88) (width 0.2) (layer "F.Cu") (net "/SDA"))
 (segment (start 147 63.54) (end 147 60.31) (width 0.2) (layer "F.Cu") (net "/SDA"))
 (segment (start 147 60.31) (end 148.31 59) (width 0.2) (layer "F.Cu") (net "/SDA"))
 (segment (start 149.7615 107.88) (end 148.2995 109.342) (width 0.2) (layer "F.Cu") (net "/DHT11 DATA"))
 (segment (start 137.021605 109.342) (end 124.679605 97) (width 0.2) (layer "F.Cu") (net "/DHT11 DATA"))
 (segment (start 148.2995 109.342) (end 137.021605 109.342) (width 0.2) (layer "F.Cu") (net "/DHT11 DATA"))
 (segment (start 113.5 92.0575) (end 117.5975 87.96) (width 0.2) (layer "F.Cu") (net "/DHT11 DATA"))
 (segment (start 124.679605 97) (end 113.5 97) (width 0.2) (layer "F.Cu") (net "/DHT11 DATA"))
 (segment (start 113.5 97) (end 113.5 92.0575) (width 0.2) (layer "F.Cu") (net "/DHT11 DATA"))
 (segment (start 144.6815 93.7915) (end 140.85 89.96) (width 0.2) (layer "F.Cu") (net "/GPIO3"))
 (segment (start 144.6815 107.88) (end 144.6815 93.7915) (width 0.2) (layer "F.Cu") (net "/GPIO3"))
 (segment (start 147.2215 107.88) (end 147.2215 101.805098) (width 0.2) (layer "F.Cu") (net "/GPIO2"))
 (segment (start 147.2215 101.805098) (end 159.066598 89.96) (width 0.2) (layer "F.Cu") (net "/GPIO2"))
 (segment (start 159.066598 89.96) (end 159.85 89.96) (width 0.2) (layer "F.Cu") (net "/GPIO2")))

